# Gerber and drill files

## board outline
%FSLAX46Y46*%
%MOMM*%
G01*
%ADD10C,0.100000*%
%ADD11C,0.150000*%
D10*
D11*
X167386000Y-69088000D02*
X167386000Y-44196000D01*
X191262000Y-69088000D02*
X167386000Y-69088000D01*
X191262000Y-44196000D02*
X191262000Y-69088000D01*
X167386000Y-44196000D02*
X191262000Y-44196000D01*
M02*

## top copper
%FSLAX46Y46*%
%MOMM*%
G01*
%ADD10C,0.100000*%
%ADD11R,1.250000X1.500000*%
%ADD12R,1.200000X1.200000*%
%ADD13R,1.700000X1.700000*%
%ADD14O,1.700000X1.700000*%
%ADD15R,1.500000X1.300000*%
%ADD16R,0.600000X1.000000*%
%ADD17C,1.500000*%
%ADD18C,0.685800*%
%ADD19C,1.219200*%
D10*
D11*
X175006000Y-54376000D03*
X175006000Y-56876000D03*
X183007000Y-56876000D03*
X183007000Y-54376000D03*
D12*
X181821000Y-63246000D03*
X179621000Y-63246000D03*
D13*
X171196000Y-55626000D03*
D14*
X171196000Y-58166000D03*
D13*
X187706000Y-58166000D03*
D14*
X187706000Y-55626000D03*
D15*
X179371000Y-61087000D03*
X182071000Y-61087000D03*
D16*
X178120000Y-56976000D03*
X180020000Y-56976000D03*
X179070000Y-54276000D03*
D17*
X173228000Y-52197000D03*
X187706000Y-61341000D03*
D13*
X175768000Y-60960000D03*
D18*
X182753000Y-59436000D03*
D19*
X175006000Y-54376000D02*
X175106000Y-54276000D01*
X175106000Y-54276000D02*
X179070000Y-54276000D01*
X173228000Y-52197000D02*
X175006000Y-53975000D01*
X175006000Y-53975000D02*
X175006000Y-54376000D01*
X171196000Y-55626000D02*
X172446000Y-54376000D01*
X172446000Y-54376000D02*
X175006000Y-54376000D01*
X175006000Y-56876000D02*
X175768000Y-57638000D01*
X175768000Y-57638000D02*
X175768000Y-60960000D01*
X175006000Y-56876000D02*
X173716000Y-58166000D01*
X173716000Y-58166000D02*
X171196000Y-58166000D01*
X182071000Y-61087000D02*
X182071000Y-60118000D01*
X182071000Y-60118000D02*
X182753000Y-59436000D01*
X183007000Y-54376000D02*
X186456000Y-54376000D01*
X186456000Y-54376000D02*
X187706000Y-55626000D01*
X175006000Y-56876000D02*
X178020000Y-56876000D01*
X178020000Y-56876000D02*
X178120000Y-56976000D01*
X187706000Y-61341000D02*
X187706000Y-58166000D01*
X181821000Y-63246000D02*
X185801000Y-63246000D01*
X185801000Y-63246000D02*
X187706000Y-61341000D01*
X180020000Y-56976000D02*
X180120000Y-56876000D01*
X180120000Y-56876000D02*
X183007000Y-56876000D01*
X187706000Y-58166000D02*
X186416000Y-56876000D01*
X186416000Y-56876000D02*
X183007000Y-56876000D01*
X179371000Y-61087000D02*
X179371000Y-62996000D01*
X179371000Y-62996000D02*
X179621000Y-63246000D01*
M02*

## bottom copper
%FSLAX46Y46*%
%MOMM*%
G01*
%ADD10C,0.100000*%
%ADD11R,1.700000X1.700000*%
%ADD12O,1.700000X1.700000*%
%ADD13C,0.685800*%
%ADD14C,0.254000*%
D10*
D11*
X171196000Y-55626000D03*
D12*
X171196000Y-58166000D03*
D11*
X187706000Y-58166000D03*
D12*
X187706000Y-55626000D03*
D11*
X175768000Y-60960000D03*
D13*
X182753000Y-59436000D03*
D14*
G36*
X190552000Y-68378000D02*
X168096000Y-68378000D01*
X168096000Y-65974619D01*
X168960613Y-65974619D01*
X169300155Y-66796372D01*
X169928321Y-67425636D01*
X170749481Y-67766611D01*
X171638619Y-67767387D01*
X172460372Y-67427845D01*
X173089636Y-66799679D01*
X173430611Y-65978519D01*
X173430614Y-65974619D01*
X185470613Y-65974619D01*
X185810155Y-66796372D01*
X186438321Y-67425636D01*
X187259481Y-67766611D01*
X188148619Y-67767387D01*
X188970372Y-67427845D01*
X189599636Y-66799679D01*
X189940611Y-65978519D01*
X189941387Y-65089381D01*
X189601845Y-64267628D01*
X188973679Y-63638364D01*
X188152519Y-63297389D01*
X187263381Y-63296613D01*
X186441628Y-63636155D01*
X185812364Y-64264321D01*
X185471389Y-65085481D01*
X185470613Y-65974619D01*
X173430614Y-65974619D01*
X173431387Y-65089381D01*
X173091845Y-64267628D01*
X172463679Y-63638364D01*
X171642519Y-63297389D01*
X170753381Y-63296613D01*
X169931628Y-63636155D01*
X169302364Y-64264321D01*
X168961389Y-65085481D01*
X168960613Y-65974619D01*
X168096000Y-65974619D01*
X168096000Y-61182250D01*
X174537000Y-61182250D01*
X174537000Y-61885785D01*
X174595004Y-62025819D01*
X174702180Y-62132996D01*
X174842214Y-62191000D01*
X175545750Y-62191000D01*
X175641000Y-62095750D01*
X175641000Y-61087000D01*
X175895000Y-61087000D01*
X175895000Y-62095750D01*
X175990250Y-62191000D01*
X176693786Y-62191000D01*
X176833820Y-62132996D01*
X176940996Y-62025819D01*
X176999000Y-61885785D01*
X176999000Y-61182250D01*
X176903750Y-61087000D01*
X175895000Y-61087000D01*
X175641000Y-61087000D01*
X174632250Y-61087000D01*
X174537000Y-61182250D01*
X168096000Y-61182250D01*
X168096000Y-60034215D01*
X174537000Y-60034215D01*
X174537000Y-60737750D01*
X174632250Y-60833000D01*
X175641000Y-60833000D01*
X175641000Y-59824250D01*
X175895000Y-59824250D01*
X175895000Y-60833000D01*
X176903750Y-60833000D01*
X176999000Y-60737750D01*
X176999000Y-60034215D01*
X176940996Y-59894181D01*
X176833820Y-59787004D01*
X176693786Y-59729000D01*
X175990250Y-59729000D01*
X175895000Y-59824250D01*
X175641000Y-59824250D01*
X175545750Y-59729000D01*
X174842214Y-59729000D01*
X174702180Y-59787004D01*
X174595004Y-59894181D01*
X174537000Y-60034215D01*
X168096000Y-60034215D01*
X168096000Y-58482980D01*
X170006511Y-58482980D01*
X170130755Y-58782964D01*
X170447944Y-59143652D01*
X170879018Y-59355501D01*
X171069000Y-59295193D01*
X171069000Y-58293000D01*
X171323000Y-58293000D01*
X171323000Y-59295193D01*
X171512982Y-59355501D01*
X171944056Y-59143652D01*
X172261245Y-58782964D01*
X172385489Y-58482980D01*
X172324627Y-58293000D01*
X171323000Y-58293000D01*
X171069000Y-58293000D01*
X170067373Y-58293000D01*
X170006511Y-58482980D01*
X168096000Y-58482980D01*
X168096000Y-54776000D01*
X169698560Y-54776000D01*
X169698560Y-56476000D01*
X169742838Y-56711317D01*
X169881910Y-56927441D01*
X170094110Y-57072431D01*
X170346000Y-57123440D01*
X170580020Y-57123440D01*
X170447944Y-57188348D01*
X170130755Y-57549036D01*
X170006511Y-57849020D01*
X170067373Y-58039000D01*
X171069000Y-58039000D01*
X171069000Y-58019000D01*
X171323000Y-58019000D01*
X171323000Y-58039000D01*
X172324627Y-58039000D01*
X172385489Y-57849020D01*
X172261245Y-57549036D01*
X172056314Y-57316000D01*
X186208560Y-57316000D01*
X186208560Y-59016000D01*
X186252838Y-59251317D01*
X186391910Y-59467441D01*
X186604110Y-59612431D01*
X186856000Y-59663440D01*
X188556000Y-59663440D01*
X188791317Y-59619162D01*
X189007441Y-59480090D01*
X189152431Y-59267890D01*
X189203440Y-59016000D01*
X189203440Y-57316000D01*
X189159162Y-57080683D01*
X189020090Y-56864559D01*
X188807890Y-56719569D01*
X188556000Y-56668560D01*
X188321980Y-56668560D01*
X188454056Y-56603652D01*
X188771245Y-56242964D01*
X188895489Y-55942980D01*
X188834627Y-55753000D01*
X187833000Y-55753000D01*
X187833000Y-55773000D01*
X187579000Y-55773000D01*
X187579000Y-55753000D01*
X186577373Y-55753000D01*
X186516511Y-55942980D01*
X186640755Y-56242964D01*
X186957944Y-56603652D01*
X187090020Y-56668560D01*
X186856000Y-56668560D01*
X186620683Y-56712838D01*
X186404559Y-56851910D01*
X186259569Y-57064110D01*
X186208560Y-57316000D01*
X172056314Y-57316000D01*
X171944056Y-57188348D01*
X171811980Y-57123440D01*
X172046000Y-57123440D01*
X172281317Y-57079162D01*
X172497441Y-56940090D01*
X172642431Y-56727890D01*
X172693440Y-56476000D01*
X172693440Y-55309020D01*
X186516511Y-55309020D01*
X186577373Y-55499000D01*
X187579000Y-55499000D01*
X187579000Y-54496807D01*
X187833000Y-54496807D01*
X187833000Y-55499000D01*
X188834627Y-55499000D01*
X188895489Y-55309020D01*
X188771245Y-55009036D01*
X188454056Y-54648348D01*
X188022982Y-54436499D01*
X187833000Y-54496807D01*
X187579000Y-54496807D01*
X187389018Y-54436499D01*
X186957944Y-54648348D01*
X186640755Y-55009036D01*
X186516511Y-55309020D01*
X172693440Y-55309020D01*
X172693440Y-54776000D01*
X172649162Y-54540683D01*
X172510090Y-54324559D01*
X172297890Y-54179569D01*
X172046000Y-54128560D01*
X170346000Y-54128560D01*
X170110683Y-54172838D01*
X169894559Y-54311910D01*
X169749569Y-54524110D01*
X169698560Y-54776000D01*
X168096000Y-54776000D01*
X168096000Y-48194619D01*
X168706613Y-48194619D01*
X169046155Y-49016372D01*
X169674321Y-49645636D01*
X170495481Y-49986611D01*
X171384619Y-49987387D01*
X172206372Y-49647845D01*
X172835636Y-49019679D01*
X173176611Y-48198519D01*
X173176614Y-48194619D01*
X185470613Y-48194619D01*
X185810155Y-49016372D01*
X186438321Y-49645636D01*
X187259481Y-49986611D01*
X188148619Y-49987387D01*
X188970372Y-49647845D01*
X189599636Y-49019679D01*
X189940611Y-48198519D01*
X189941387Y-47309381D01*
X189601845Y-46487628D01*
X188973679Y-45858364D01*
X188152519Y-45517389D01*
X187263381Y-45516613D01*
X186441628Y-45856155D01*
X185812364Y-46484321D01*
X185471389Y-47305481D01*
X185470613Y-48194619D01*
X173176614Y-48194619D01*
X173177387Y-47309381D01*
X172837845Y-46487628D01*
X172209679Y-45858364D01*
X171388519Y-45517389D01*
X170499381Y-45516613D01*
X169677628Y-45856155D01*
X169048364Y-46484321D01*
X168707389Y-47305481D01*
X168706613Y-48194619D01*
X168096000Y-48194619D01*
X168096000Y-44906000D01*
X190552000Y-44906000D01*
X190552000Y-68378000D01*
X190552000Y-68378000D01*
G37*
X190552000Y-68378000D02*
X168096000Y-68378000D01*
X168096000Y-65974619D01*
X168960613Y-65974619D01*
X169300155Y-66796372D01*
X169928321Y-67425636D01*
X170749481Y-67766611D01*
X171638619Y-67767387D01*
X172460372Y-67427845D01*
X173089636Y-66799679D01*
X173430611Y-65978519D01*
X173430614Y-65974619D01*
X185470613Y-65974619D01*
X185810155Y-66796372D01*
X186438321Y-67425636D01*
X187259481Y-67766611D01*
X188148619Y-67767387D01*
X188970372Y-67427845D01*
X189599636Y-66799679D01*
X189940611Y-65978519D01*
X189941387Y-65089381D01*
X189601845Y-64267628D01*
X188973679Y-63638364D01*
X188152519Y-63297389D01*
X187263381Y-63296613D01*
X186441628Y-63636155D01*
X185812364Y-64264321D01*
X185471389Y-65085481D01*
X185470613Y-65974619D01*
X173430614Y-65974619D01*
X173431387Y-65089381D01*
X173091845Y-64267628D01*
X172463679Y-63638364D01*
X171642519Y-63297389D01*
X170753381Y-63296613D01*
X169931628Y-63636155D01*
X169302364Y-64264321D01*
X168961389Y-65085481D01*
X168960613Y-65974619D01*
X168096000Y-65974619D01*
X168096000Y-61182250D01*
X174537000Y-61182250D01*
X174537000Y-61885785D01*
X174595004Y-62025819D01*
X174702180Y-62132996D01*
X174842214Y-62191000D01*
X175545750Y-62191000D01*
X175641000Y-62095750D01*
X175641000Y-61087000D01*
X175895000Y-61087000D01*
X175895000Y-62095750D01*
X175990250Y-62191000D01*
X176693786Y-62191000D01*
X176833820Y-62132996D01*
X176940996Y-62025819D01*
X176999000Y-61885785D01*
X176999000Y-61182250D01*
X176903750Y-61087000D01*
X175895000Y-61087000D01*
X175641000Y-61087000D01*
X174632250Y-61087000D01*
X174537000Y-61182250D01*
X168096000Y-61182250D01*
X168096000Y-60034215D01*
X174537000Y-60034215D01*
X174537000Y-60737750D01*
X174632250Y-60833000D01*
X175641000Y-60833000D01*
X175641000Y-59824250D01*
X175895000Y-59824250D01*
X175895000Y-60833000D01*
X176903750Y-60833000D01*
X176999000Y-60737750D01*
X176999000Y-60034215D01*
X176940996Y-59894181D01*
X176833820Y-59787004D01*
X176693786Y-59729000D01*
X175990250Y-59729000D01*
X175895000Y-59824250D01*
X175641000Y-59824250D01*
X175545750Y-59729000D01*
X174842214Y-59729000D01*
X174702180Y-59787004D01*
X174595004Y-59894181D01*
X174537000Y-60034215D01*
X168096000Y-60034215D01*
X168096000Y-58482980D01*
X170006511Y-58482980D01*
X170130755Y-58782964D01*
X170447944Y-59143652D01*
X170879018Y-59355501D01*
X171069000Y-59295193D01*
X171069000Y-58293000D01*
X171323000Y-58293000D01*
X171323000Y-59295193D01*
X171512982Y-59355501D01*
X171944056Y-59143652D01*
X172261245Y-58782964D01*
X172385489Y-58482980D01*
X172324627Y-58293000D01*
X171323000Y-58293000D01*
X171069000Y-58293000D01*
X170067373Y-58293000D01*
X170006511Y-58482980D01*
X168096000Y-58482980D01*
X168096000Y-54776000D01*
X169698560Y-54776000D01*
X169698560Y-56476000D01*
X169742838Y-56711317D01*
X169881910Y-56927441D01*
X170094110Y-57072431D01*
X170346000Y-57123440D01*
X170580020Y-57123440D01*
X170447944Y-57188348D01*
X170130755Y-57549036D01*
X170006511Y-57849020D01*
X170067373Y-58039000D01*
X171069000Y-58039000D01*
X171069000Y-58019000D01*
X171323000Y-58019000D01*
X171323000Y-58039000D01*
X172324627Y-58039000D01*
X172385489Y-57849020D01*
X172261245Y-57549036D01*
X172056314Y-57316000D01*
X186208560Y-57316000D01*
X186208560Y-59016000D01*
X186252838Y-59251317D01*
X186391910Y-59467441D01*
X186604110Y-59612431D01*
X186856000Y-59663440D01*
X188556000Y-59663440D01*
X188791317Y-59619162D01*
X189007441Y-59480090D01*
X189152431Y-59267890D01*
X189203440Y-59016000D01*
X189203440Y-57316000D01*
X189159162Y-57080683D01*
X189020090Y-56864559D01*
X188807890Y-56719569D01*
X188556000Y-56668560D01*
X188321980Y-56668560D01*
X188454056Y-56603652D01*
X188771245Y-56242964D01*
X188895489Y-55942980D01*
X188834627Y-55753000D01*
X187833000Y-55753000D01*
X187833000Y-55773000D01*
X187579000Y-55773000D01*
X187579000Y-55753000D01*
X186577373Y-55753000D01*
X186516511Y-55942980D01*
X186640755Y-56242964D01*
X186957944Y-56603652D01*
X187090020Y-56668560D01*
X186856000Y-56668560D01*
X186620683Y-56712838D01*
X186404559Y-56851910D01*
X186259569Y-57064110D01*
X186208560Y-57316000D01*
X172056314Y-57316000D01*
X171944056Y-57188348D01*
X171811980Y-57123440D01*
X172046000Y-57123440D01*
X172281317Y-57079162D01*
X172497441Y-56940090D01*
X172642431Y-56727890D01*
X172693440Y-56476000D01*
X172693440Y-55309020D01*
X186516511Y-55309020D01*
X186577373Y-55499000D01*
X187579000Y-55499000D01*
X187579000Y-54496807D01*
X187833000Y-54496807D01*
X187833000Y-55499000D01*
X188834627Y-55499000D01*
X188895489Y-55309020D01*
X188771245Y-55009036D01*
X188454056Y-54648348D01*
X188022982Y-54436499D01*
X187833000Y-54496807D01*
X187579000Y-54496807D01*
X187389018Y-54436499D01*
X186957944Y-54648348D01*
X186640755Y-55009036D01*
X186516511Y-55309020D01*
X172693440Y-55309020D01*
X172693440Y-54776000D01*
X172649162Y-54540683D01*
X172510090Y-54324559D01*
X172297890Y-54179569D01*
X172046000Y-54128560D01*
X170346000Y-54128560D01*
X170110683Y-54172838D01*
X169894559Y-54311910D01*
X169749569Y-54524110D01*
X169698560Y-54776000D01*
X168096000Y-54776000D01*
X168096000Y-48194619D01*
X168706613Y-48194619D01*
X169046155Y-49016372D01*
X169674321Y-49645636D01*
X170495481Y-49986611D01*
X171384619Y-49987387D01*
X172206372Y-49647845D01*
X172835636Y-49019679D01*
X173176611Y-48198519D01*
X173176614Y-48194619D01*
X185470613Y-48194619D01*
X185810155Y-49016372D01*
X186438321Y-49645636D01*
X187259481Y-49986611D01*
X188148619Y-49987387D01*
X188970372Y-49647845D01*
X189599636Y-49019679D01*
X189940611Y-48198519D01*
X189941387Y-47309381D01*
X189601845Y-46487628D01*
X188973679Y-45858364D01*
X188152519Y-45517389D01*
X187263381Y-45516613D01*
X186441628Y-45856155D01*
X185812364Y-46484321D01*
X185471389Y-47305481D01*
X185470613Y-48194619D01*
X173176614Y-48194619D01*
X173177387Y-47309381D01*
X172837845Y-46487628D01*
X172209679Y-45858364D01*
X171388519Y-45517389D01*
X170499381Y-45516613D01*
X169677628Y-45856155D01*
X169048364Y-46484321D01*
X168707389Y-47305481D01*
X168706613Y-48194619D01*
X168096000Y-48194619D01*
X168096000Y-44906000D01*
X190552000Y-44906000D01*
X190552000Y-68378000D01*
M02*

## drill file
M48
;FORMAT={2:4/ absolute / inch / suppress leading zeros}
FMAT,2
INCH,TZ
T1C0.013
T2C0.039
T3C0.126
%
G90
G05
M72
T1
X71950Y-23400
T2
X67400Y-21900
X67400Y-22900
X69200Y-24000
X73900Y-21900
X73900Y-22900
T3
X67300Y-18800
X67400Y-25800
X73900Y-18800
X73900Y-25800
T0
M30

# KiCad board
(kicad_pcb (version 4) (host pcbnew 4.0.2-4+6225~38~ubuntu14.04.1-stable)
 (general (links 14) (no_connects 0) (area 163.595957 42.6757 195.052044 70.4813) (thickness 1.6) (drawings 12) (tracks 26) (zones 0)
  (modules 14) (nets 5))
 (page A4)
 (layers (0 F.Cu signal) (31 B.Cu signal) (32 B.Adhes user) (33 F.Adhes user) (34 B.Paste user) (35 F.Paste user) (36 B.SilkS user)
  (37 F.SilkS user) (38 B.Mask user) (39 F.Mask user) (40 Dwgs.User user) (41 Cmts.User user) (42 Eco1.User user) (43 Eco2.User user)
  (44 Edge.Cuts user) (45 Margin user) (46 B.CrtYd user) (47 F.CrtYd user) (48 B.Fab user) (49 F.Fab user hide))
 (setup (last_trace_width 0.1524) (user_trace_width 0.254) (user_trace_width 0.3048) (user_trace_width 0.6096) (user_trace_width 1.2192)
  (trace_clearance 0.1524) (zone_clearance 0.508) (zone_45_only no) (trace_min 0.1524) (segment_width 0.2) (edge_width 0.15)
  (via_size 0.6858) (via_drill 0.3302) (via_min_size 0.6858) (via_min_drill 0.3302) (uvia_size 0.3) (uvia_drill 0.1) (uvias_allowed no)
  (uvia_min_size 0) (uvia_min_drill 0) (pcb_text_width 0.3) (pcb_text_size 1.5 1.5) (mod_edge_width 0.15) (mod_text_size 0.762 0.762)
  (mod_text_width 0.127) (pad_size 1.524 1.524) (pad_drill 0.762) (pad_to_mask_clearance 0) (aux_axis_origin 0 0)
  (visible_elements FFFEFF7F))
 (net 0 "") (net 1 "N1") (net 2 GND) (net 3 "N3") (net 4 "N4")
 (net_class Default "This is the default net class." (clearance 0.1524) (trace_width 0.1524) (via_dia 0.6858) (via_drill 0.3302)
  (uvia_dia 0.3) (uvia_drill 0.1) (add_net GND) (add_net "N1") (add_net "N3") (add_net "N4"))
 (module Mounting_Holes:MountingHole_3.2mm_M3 (layer F.Cu) (at 187.706 65.532)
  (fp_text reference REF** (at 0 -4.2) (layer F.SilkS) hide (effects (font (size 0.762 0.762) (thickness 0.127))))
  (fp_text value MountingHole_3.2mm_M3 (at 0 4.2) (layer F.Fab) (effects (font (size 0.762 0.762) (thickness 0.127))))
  (pad 1 np_thru_hole circle (at 0 0) (size 3.2 3.2) (drill 3.2) (layers *.Cu *.Mask)))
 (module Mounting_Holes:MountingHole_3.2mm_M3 (layer F.Cu) (at 170.942 47.752)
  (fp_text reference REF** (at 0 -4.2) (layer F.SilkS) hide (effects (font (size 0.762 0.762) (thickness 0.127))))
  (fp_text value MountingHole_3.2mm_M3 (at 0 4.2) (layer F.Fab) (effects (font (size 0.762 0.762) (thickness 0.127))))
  (pad 1 np_thru_hole circle (at 0 0) (size 3.2 3.2) (drill 3.2) (layers *.Cu *.Mask)))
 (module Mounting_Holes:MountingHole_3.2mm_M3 (layer F.Cu) (at 171.196 65.532)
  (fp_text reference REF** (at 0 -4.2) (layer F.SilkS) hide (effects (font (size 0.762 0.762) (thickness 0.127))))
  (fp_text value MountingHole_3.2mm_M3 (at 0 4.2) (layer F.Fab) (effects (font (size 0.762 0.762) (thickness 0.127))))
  (pad 1 np_thru_hole circle (at 0 0) (size 3.2 3.2) (drill 3.2) (layers *.Cu *.Mask)))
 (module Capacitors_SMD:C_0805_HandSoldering (layer F.Cu) (at 175.006 55.626 270)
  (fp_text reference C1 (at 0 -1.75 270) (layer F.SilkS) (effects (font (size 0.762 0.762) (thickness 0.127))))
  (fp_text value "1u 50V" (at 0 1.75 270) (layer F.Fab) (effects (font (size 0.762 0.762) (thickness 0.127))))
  (pad 1 smd rect (at -1.25 0 270) (size 1.5 1.25) (layers F.Cu F.Paste F.Mask) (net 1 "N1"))
  (pad 2 smd rect (at 1.25 0 270) (size 1.5 1.25) (layers F.Cu F.Paste F.Mask) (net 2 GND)))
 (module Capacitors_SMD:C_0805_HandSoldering (layer F.Cu) (at 183.007 55.626 90)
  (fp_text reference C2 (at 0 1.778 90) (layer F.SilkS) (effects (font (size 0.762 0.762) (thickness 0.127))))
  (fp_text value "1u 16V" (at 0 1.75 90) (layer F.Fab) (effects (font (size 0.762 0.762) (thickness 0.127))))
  (pad 1 smd rect (at -1.25 0 90) (size 1.5 1.25) (layers F.Cu F.Paste F.Mask) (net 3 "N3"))
  (pad 2 smd rect (at 1.25 0 90) (size 1.5 1.25) (layers F.Cu F.Paste F.Mask) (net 2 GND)))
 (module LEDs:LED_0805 (layer F.Cu) (at 180.721 63.246)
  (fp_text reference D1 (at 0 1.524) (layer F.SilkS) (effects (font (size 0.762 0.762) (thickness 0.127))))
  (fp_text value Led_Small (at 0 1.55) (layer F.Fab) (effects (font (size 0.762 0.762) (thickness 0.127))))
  (pad 2 smd rect (at 1.1 0 180) (size 1.2 1.2) (layers F.Cu F.Paste F.Mask) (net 3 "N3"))
  (pad 1 smd rect (at -1.1 0 180) (size 1.2 1.2) (layers F.Cu F.Paste F.Mask) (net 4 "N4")))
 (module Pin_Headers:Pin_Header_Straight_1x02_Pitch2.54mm (layer F.Cu) (at 171.196 55.626)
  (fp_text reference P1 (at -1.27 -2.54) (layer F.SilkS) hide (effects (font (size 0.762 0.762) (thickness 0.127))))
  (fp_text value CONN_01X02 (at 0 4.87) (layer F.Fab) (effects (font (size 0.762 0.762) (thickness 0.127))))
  (pad 1 thru_hole rect (at 0 0) (size 1.7 1.7) (drill 1) (layers *.Cu *.Mask) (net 1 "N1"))
  (pad 2 thru_hole oval (at 0 2.54) (size 1.7 1.7) (drill 1) (layers *.Cu *.Mask) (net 2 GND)))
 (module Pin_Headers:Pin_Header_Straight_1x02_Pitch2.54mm (layer F.Cu) (at 187.706 58.166 180)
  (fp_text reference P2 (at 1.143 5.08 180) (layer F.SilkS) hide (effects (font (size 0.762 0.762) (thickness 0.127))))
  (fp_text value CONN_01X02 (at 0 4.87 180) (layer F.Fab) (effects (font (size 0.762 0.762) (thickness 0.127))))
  (pad 1 thru_hole rect (at 0 0 180) (size 1.7 1.7) (drill 1) (layers *.Cu *.Mask) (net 3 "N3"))
  (pad 2 thru_hole oval (at 0 2.54 180) (size 1.7 1.7) (drill 1) (layers *.Cu *.Mask) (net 2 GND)))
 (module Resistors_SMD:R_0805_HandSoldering (layer F.Cu) (at 180.721 61.087)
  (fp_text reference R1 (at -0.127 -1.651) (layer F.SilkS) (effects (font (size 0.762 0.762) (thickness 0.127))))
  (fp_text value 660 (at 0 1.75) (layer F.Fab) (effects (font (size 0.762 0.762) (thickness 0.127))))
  (pad 1 smd rect (at -1.35 0) (size 1.5 1.3) (layers F.Cu F.Paste F.Mask) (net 4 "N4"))
  (pad 2 smd rect (at 1.35 0) (size 1.5 1.3) (layers F.Cu F.Paste F.Mask) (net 2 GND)))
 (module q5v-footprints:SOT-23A (layer F.Cu) (at 179.07 55.626)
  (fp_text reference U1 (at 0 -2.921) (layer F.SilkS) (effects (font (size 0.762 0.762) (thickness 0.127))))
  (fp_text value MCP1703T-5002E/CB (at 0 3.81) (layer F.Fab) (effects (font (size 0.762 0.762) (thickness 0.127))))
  (pad 1 smd rect (at -0.95 1.35) (size 0.6 1) (layers F.Cu F.Paste F.Mask) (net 2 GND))
  (pad 2 smd rect (at 0.95 1.35) (size 0.6 1) (layers F.Cu F.Paste F.Mask) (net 3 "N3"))
  (pad 3 smd rect (at 0 -1.35) (size 0.6 1) (layers F.Cu F.Paste F.Mask) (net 1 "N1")))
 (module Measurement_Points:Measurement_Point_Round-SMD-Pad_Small (layer F.Cu) (at 173.228 52.197)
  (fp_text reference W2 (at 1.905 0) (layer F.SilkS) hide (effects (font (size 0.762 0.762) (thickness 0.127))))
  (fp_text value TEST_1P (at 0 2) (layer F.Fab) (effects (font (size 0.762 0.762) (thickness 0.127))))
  (pad 1 smd circle (at 0 0) (size 1.5 1.5) (layers F.Cu F.Mask) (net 1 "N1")))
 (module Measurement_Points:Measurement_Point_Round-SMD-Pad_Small (layer F.Cu) (at 187.706 61.341)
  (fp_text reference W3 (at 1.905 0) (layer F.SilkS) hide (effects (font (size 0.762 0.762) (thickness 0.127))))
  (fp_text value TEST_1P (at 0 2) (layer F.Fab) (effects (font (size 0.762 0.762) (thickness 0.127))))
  (pad 1 smd circle (at 0 0) (size 1.5 1.5) (layers F.Cu F.Mask) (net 3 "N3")))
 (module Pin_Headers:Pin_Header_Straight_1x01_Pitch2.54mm (layer F.Cu) (at 175.768 60.96)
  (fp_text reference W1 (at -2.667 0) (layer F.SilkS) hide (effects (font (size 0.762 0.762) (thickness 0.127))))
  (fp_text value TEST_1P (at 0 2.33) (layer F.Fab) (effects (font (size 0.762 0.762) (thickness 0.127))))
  (pad 1 thru_hole rect (at 0 0) (size 1.7 1.7) (drill 1) (layers *.Cu *.Mask) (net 2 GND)))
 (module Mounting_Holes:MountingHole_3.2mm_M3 (layer F.Cu) (at 187.706 47.752)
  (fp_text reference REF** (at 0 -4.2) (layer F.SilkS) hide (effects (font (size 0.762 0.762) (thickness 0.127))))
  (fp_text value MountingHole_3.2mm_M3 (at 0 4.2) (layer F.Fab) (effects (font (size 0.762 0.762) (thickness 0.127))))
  (pad 1 np_thru_hole circle (at 0 0) (size 3.2 3.2) (drill 3.2) (layers *.Cu *.Mask)))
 (gr_line (start 167.386 69.088) (end 167.386 44.196) (angle 90) (layer Edge.Cuts) (width 0.15))
 (gr_line (start 191.262 69.088) (end 167.386 69.088) (angle 90) (layer Edge.Cuts) (width 0.15))
 (gr_line (start 191.262 44.196) (end 191.262 69.088) (angle 90) (layer Edge.Cuts) (width 0.15))
 (gr_line (start 167.386 44.196) (end 191.262 44.196) (angle 90) (layer Edge.Cuts) (width 0.15))
 (segment (start 175.006 54.376) (end 175.106 54.276) (width 1.2192) (layer F.Cu) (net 1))
 (segment (start 175.106 54.276) (end 179.07 54.276) (width 1.2192) (layer F.Cu) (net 1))
 (segment (start 173.228 52.197) (end 175.006 53.975) (width 1.2192) (layer F.Cu) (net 1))
 (segment (start 175.006 53.975) (end 175.006 54.376) (width 1.2192) (layer F.Cu) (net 1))
 (segment (start 171.196 55.626) (end 172.446 54.376) (width 1.2192) (layer F.Cu) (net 1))
 (segment (start 172.446 54.376) (end 175.006 54.376) (width 1.2192) (layer F.Cu) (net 1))
 (segment (start 175.006 56.876) (end 175.768 57.638) (width 1.2192) (layer F.Cu) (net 2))
 (segment (start 175.768 57.638) (end 175.768 60.96) (width 1.2192) (layer F.Cu) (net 2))
 (segment (start 175.006 56.876) (end 173.716 58.166) (width 1.2192) (layer F.Cu) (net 2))
 (segment (start 173.716 58.166) (end 171.196 58.166) (width 1.2192) (layer F.Cu) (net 2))
 (segment (start 182.071 61.087) (end 182.071 60.118) (width 1.2192) (layer F.Cu) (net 2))
 (via (at 182.753 59.436) (size 0.6858) (drill 0.3302) (layers F.Cu B.Cu) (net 2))
 (segment (start 182.071 60.118) (end 182.753 59.436) (width 1.2192) (layer F.Cu) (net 2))
 (segment (start 183.007 54.376) (end 186.456 54.376) (width 1.2192) (layer F.Cu) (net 2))
 (segment (start 186.456 54.376) (end 187.706 55.626) (width 1.2192) (layer F.Cu) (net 2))
 (segment (start 175.006 56.876) (end 178.02 56.876) (width 1.2192) (layer F.Cu) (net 2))
 (segment (start 178.02 56.876) (end 178.12 56.976) (width 1.2192) (layer F.Cu) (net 2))
 (segment (start 187.706 61.341) (end 187.706 58.166) (width 1.2192) (layer F.Cu) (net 3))
 (segment (start 181.821 63.246) (end 185.801 63.246) (width 1.2192) (layer F.Cu) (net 3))
 (segment (start 185.801 63.246) (end 187.706 61.341) (width 1.2192) (layer F.Cu) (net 3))
 (segment (start 180.02 56.976) (end 180.12 56.876) (width 1.2192) (layer F.Cu) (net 3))
 (segment (start 180.12 56.876) (end 183.007 56.876) (width 1.2192) (layer F.Cu) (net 3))
 (segment (start 187.706 58.166) (end 186.416 56.876) (width 1.2192) (layer F.Cu) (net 3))
 (segment (start 186.416 56.876) (end 183.007 56.876) (width 1.2192) (layer F.Cu) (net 3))
 (segment (start 179.371 61.087) (end 179.371 62.996) (width 1.2192) (layer F.Cu) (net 4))
 (segment (start 179.371 62.996) (end 179.621 63.246) (width 1.2192) (layer F.Cu) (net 4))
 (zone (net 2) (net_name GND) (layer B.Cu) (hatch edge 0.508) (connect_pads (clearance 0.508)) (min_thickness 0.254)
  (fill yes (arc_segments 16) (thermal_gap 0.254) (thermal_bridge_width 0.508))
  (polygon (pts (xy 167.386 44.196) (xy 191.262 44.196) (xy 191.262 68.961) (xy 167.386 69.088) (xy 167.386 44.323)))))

